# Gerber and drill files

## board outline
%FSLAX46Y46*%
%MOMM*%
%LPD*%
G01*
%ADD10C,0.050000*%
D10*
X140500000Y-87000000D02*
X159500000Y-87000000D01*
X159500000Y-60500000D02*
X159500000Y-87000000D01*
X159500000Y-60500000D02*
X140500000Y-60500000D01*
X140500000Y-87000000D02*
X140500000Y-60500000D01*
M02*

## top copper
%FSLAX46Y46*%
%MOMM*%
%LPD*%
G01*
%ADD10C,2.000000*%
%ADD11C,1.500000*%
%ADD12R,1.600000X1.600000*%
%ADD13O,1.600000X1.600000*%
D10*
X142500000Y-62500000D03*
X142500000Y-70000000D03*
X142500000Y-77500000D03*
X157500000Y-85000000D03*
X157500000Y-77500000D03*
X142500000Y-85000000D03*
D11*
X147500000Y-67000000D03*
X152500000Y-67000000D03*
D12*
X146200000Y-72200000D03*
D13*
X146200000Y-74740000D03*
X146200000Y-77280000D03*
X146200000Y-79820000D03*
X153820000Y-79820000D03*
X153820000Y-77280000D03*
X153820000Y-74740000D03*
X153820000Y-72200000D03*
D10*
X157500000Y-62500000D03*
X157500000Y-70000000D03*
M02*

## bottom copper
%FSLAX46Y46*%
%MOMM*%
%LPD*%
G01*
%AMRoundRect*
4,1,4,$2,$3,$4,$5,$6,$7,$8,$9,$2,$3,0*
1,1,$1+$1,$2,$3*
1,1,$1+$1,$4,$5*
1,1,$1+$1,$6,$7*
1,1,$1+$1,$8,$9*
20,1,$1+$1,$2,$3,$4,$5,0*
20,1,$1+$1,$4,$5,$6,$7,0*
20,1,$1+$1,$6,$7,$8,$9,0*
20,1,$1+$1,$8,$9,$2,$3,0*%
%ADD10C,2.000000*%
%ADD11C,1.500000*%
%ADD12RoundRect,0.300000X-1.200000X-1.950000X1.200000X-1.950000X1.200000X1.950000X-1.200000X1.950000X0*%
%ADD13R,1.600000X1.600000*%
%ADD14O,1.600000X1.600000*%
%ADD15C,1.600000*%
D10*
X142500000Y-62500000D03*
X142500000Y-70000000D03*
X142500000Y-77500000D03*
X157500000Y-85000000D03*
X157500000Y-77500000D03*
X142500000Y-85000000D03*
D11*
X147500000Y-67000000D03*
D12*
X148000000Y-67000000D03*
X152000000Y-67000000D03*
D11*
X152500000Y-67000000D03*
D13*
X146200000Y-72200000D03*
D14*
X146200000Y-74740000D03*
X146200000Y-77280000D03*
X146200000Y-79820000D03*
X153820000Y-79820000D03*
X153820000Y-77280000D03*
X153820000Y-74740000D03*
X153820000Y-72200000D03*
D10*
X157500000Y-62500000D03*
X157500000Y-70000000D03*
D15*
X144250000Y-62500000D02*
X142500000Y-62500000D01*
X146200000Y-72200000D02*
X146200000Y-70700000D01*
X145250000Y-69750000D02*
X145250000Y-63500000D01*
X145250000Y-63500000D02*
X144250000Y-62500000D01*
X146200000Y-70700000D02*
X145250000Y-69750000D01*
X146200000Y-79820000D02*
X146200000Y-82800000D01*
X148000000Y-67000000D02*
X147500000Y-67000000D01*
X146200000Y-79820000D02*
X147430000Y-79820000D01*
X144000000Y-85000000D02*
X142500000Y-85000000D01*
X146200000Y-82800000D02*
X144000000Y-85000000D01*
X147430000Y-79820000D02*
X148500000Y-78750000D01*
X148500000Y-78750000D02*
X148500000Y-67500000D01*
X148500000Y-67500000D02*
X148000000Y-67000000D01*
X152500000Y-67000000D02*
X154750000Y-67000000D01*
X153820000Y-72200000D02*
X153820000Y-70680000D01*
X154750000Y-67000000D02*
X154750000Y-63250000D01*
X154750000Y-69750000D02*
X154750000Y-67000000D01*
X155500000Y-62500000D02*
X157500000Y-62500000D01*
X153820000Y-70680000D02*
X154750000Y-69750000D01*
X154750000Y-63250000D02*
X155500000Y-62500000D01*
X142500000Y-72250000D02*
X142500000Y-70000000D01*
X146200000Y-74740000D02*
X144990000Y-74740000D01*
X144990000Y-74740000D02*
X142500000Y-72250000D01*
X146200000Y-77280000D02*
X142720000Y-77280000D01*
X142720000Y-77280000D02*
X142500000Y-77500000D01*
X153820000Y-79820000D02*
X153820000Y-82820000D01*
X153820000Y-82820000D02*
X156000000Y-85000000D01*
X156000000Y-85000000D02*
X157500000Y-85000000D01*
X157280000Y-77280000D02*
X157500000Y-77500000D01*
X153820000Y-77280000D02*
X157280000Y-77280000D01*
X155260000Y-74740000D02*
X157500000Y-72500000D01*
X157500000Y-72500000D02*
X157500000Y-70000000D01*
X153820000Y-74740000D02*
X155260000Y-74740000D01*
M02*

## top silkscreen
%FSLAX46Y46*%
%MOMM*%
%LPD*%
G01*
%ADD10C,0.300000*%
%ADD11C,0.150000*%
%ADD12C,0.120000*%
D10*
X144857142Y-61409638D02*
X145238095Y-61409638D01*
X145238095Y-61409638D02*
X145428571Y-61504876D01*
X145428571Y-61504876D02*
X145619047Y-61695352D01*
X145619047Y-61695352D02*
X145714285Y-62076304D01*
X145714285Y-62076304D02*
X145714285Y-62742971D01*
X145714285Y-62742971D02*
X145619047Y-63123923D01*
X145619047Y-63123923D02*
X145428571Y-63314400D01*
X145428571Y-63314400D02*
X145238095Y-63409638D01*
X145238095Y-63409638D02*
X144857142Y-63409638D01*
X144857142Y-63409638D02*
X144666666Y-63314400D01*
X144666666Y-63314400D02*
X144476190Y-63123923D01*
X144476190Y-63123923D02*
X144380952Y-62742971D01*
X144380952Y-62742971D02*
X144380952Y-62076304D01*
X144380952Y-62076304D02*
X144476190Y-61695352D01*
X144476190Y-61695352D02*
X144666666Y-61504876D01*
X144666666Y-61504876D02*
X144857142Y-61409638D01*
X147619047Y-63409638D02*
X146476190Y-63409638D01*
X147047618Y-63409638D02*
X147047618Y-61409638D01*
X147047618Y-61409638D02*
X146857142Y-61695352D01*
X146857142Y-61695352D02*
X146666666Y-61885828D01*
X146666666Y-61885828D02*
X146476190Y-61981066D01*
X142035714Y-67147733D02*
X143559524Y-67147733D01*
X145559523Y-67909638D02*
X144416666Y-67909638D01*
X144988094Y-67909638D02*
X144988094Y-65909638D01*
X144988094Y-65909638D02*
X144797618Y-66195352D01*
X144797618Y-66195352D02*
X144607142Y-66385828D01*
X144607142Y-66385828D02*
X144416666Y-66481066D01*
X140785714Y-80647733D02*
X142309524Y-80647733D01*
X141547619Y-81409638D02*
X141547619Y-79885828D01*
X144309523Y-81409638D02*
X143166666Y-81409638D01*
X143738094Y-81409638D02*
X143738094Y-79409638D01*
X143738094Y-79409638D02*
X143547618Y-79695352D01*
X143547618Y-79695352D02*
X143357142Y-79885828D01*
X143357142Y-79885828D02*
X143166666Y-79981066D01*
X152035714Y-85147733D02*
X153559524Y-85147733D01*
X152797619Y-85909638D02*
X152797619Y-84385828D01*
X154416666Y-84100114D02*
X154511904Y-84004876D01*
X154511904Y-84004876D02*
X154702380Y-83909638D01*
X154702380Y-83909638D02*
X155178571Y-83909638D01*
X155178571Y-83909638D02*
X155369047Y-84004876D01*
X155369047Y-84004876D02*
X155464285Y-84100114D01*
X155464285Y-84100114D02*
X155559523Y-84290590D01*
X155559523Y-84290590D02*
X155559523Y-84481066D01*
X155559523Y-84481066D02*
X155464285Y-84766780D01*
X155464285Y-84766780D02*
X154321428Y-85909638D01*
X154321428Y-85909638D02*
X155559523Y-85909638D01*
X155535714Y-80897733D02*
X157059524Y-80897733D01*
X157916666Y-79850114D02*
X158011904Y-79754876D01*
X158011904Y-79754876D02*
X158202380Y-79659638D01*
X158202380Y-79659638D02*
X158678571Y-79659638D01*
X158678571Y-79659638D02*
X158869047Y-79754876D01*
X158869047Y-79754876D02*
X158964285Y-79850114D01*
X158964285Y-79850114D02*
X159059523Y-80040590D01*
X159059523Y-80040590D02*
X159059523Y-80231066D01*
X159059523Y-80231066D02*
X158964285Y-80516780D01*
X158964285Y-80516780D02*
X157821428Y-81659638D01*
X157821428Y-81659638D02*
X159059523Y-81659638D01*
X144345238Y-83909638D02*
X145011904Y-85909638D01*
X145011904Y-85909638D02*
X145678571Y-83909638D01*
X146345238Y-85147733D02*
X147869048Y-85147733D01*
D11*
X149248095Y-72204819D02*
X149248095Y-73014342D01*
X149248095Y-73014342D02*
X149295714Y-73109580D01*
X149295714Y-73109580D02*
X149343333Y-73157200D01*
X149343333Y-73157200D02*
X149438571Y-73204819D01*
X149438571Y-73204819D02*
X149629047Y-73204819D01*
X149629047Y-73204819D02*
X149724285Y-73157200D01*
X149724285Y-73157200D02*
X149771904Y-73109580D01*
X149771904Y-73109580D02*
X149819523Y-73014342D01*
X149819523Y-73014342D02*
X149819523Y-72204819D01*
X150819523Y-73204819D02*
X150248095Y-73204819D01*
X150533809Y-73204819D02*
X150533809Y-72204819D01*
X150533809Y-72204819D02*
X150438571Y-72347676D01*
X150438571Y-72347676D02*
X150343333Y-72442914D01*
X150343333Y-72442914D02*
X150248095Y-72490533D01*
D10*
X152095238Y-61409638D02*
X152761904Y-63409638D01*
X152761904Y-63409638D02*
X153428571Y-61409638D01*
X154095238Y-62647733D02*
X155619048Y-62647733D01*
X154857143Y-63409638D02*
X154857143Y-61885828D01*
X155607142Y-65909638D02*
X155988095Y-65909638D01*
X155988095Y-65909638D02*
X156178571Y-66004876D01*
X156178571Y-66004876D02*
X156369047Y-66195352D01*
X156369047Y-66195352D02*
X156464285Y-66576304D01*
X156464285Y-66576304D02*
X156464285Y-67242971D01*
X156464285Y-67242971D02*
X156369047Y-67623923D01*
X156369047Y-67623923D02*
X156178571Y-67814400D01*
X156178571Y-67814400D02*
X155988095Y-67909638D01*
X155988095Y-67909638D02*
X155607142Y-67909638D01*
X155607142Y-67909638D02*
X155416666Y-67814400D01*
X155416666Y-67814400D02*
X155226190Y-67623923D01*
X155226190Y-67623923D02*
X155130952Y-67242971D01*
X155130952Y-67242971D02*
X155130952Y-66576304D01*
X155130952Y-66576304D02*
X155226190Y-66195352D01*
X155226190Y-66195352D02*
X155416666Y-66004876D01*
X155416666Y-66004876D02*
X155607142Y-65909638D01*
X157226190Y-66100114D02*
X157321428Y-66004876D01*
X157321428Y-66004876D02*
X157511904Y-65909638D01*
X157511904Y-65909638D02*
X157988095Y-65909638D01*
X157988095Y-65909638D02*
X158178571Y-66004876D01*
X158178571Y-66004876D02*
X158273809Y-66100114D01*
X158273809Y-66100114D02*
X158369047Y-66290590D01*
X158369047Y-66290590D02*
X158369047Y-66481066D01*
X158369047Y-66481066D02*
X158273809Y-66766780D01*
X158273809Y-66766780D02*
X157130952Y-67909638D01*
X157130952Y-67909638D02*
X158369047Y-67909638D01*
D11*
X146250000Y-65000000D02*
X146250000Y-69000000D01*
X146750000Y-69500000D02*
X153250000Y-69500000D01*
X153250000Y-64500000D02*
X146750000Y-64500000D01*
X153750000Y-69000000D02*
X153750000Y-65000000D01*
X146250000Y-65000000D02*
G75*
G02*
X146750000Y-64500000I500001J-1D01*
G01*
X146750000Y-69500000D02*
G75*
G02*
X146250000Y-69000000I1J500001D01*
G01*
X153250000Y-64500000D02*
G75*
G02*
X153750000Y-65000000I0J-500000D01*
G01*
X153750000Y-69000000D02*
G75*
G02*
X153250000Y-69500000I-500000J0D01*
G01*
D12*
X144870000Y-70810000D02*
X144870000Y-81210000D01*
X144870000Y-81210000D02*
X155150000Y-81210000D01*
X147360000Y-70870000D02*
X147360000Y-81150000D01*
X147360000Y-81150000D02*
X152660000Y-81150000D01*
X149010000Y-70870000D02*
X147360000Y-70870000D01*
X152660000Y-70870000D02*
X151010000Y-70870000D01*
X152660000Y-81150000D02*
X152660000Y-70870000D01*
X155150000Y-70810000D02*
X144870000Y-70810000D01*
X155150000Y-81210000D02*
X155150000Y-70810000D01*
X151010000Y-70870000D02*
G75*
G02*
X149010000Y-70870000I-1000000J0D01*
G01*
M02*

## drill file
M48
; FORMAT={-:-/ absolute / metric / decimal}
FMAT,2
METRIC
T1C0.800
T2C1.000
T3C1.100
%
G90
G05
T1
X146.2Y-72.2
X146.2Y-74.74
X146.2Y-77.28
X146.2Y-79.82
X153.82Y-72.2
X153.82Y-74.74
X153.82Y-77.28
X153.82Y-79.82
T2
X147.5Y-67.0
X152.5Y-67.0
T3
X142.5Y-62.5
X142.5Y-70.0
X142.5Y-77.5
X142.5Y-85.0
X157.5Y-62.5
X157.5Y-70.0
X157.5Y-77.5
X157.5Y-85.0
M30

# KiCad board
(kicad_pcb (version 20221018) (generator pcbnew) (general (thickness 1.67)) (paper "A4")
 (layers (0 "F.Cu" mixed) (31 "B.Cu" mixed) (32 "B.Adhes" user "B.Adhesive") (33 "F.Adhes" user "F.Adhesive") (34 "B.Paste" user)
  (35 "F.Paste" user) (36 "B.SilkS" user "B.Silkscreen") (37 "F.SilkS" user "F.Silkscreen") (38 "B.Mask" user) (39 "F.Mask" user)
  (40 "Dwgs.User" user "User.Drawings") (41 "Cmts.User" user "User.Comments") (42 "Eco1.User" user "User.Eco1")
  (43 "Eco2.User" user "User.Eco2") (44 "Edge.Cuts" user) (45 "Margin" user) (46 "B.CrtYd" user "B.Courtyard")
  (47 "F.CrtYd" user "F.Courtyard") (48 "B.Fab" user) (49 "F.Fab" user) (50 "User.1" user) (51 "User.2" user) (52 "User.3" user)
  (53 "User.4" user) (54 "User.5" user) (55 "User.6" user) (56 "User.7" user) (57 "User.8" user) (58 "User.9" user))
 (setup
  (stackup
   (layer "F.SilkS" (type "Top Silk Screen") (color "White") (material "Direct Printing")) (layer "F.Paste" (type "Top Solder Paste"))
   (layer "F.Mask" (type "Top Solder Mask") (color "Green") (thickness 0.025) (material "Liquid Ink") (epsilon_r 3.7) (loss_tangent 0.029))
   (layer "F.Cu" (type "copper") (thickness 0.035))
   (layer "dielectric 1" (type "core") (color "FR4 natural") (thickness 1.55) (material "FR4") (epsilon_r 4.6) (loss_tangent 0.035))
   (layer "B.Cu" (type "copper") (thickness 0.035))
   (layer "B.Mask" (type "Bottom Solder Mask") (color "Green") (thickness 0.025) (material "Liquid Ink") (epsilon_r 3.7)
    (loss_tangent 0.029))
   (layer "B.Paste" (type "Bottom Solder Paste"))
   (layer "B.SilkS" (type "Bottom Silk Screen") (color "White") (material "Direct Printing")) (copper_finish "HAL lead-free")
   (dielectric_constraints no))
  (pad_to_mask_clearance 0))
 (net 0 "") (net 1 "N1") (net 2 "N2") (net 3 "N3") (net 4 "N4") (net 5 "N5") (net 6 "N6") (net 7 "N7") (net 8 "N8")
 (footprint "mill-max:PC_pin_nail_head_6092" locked (layer "F.Cu") (at 142.5 62.5)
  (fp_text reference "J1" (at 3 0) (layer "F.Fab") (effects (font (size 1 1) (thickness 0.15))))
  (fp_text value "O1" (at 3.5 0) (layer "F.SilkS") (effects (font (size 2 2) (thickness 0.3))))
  (pad "1" thru_hole circle locked (at 0 0) (size 2 2) (drill 1.1) (layers "*.Cu" "*.Mask") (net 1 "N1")))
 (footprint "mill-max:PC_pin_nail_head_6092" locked (layer "F.Cu") (at 142.5 70)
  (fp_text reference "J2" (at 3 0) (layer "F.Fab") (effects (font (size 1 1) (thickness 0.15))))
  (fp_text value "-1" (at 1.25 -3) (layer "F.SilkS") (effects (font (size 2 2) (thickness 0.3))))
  (pad "1" thru_hole circle locked (at 0 0) (size 2 2) (drill 1.1) (layers "*.Cu" "*.Mask") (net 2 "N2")))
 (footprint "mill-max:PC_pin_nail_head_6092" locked (layer "F.Cu") (at 142.5 77.5)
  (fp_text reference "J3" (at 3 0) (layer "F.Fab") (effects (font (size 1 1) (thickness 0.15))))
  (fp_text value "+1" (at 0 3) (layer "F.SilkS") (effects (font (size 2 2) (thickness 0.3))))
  (pad "1" thru_hole circle locked (at 0 0) (size 2 2) (drill 1.1) (layers "*.Cu" "*.Mask") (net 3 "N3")))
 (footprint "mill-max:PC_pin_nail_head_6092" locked (layer "F.Cu") (at 157.5 85)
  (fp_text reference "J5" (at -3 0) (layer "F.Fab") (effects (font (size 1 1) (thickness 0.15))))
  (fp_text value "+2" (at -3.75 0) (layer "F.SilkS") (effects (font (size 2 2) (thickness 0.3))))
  (pad "1" thru_hole circle locked (at 0 0) (size 2 2) (drill 1.1) (layers "*.Cu" "*.Mask") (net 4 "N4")))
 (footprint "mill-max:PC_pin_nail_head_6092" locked (layer "F.Cu") (at 157.5 77.5)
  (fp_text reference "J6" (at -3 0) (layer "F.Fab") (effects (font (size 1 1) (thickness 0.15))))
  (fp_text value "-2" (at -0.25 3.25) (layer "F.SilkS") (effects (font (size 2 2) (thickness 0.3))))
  (pad "1" thru_hole circle locked (at 0 0) (size 2 2) (drill 1.1) (layers "*.Cu" "*.Mask") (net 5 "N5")))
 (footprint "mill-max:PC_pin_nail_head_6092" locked (layer "F.Cu") (at 142.5 85 180)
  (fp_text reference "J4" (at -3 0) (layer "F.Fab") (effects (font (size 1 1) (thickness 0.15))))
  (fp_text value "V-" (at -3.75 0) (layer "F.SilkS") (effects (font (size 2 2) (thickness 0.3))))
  (pad "1" thru_hole circle locked (at 0 0 180) (size 2 2) (drill 1.1) (layers "*.Cu" "*.Mask") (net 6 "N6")))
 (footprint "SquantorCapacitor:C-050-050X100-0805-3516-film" (layer "F.Cu") (at 150 67)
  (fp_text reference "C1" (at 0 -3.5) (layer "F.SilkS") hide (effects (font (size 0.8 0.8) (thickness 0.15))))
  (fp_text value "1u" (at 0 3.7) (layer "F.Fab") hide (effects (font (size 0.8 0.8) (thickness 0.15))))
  (fp_line (start -3.75 -2) (end -3.75 2) (stroke (width 0.15) (type solid)) (layer "F.SilkS"))
  (fp_line (start -3.25 2.5) (end 3.25 2.5) (stroke (width 0.15) (type solid)) (layer "F.SilkS"))
  (fp_line (start 3.25 -2.5) (end -3.25 -2.5) (stroke (width 0.15) (type solid)) (layer "F.SilkS"))
  (fp_line (start 3.75 2) (end 3.75 -2) (stroke (width 0.15) (type solid)) (layer "F.SilkS"))
  (fp_arc (start -3.75 -2) (mid -3.603553 -2.353553) (end -3.25 -2.5) (stroke (width 0.15) (type solid)) (layer "F.SilkS"))
  (fp_arc (start -3.25 2.5) (mid -3.603553 2.353553) (end -3.75 2) (stroke (width 0.15) (type solid)) (layer "F.SilkS"))
  (fp_arc (start 3.25 -2.5) (mid 3.603553 -2.353553) (end 3.75 -2) (stroke (width 0.15) (type solid)) (layer "F.SilkS"))
  (fp_arc (start 3.75 2) (mid 3.603553 2.353553) (end 3.25 2.5) (stroke (width 0.15) (type solid)) (layer "F.SilkS"))
  (pad "1" thru_hole circle (at -2.5 0) (size 1.5 1.5) (drill 1) (layers "*.Cu" "*.Mask") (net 6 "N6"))
  (pad "1" smd roundrect (at -2 0) (size 3 4.5) (layers "B.Cu" "B.Paste" "B.Mask") (roundrect_rratio 0.1) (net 6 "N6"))
  (pad "2" smd roundrect (at 2 0) (size 3 4.5) (layers "B.Cu" "B.Paste" "B.Mask") (roundrect_rratio 0.1) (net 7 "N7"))
  (pad "2" thru_hole circle (at 2.5 0) (size 1.5 1.5) (drill 1) (layers "*.Cu" "*.Mask") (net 7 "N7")))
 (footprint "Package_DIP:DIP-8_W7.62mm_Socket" (layer "F.Cu") (at 146.2 72.2)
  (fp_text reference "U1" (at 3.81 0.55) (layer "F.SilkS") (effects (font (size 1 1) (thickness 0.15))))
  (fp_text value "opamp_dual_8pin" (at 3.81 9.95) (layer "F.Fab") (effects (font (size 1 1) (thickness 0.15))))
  (fp_line (start -1.33 -1.39) (end -1.33 9.01) (stroke (width 0.12) (type solid)) (layer "F.SilkS"))
  (fp_line (start -1.33 9.01) (end 8.95 9.01) (stroke (width 0.12) (type solid)) (layer "F.SilkS"))
  (fp_line (start 1.16 -1.33) (end 1.16 8.95) (stroke (width 0.12) (type solid)) (layer "F.SilkS"))
  (fp_line (start 1.16 8.95) (end 6.46 8.95) (stroke (width 0.12) (type solid)) (layer "F.SilkS"))
  (fp_line (start 2.81 -1.33) (end 1.16 -1.33) (stroke (width 0.12) (type solid)) (layer "F.SilkS"))
  (fp_line (start 6.46 -1.33) (end 4.81 -1.33) (stroke (width 0.12) (type solid)) (layer "F.SilkS"))
  (fp_line (start 6.46 8.95) (end 6.46 -1.33) (stroke (width 0.12) (type solid)) (layer "F.SilkS"))
  (fp_line (start 8.95 -1.39) (end -1.33 -1.39) (stroke (width 0.12) (type solid)) (layer "F.SilkS"))
  (fp_line (start 8.95 9.01) (end 8.95 -1.39) (stroke (width 0.12) (type solid)) (layer "F.SilkS"))
  (fp_arc (start 4.81 -1.33) (mid 3.81 -0.33) (end 2.81 -1.33) (stroke (width 0.12) (type solid)) (layer "F.SilkS"))
  (pad "1" thru_hole rect (at 0 0) (size 1.6 1.6) (drill 0.8) (layers "*.Cu" "*.Mask") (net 1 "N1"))
  (pad "2" thru_hole oval (at 0 2.54) (size 1.6 1.6) (drill 0.8) (layers "*.Cu" "*.Mask") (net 2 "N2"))
  (pad "3" thru_hole oval (at 0 5.08) (size 1.6 1.6) (drill 0.8) (layers "*.Cu" "*.Mask") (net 3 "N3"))
  (pad "4" thru_hole oval (at 0 7.62) (size 1.6 1.6) (drill 0.8) (layers "*.Cu" "*.Mask") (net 6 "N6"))
  (pad "5" thru_hole oval (at 7.62 7.62) (size 1.6 1.6) (drill 0.8) (layers "*.Cu" "*.Mask") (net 4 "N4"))
  (pad "6" thru_hole oval (at 7.62 5.08) (size 1.6 1.6) (drill 0.8) (layers "*.Cu" "*.Mask") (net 5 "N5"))
  (pad "7" thru_hole oval (at 7.62 2.54) (size 1.6 1.6) (drill 0.8) (layers "*.Cu" "*.Mask") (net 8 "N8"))
  (pad "8" thru_hole oval (at 7.62 0) (size 1.6 1.6) (drill 0.8) (layers "*.Cu" "*.Mask") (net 7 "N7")))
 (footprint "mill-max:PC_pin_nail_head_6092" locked (layer "F.Cu") (at 157.5 62.5)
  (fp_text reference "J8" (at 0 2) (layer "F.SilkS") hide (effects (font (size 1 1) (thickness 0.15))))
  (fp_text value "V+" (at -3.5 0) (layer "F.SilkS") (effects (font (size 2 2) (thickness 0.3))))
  (pad "1" thru_hole circle locked (at 0 0) (size 2 2) (drill 1.1) (layers "*.Cu" "*.Mask") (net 7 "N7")))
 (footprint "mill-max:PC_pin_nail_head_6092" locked (layer "F.Cu") (at 157.5 70)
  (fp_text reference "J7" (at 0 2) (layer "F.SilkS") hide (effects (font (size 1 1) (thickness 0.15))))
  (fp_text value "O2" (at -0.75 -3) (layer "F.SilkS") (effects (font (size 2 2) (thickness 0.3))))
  (pad "1" thru_hole circle locked (at 0 0) (size 2 2) (drill 1.1) (layers "*.Cu" "*.Mask") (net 8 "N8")))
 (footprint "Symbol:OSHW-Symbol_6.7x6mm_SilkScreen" (layer "B.Cu") (at 149.5 82.55 180)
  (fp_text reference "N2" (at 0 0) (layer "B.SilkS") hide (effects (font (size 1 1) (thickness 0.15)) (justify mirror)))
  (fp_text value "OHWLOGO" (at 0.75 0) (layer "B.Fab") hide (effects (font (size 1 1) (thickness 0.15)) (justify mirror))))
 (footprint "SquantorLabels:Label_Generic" (layer "B.Cu") (at 150.4 86.25 180)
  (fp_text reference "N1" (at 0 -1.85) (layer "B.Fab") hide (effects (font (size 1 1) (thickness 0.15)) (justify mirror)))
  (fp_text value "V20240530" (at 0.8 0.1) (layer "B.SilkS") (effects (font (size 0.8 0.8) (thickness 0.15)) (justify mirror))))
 (gr_line (start 140.5 87) (end 159.5 87) (stroke (width 0.05) (type solid)) (layer "Edge.Cuts"))
 (gr_line (start 159.5 60.5) (end 159.5 87) (stroke (width 0.05) (type solid)) (layer "Edge.Cuts"))
 (gr_line (start 159.5 60.5) (end 140.5 60.5) (stroke (width 0.05) (type solid)) (layer "Edge.Cuts"))
 (gr_line (start 140.5 87) (end 140.5 60.5) (stroke (width 0.05) (type solid)) (layer "Edge.Cuts"))
 (segment (start 144.25 62.5) (end 142.5 62.5) (width 1.6) (layer "B.Cu") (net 1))
 (segment (start 146.2 72.2) (end 146.2 70.7) (width 1.6) (layer "B.Cu") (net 1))
 (segment (start 145.25 69.75) (end 145.25 63.5) (width 1.6) (layer "B.Cu") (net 1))
 (segment (start 145.25 63.5) (end 144.25 62.5) (width 1.6) (layer "B.Cu") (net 1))
 (segment (start 146.2 70.7) (end 145.25 69.75) (width 1.6) (layer "B.Cu") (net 1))
 (segment (start 146.2 79.82) (end 146.2 82.8) (width 1.6) (layer "B.Cu") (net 6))
 (segment (start 148 67) (end 147.5 67) (width 1.6) (layer "B.Cu") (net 6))
 (segment (start 146.2 79.82) (end 147.43 79.82) (width 1.6) (layer "B.Cu") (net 6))
 (segment (start 144 85) (end 142.5 85) (width 1.6) (layer "B.Cu") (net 6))
 (segment (start 146.2 82.8) (end 144 85) (width 1.6) (layer "B.Cu") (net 6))
 (segment (start 147.43 79.82) (end 148.5 78.75) (width 1.6) (layer "B.Cu") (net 6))
 (segment (start 148.5 78.75) (end 148.5 67.5) (width 1.6) (layer "B.Cu") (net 6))
 (segment (start 148.5 67.5) (end 148 67) (width 1.6) (layer "B.Cu") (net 6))
 (segment (start 152.5 67) (end 154.75 67) (width 1.6) (layer "B.Cu") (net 7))
 (segment (start 153.82 72.2) (end 153.82 70.68) (width 1.6) (layer "B.Cu") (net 7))
 (segment (start 154.75 67) (end 154.75 63.25) (width 1.6) (layer "B.Cu") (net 7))
 (segment (start 154.75 69.75) (end 154.75 67) (width 1.6) (layer "B.Cu") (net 7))
 (segment (start 155.5 62.5) (end 157.5 62.5) (width 1.6) (layer "B.Cu") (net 7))
 (segment (start 153.82 70.68) (end 154.75 69.75) (width 1.6) (layer "B.Cu") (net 7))
 (segment (start 154.75 63.25) (end 155.5 62.5) (width 1.6) (layer "B.Cu") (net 7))
 (segment (start 142.5 72.25) (end 142.5 70) (width 1.6) (layer "B.Cu") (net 2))
 (segment (start 146.2 74.74) (end 144.99 74.74) (width 1.6) (layer "B.Cu") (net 2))
 (segment (start 144.99 74.74) (end 142.5 72.25) (width 1.6) (layer "B.Cu") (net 2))
 (segment (start 146.2 77.28) (end 142.72 77.28) (width 1.6) (layer "B.Cu") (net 3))
 (segment (start 142.72 77.28) (end 142.5 77.5) (width 1.6) (layer "B.Cu") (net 3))
 (segment (start 153.82 79.82) (end 153.82 82.82) (width 1.6) (layer "B.Cu") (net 4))
 (segment (start 153.82 82.82) (end 156 85) (width 1.6) (layer "B.Cu") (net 4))
 (segment (start 156 85) (end 157.5 85) (width 1.6) (layer "B.Cu") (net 4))
 (segment (start 157.28 77.28) (end 157.5 77.5) (width 1.6) (layer "B.Cu") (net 5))
 (segment (start 153.82 77.28) (end 157.28 77.28) (width 1.6) (layer "B.Cu") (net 5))
 (segment (start 155.26 74.74) (end 157.5 72.5) (width 1.6) (layer "B.Cu") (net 8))
 (segment (start 157.5 72.5) (end 157.5 70) (width 1.6) (layer "B.Cu") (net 8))
 (segment (start 153.82 74.74) (end 155.26 74.74) (width 1.6) (layer "B.Cu") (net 8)))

